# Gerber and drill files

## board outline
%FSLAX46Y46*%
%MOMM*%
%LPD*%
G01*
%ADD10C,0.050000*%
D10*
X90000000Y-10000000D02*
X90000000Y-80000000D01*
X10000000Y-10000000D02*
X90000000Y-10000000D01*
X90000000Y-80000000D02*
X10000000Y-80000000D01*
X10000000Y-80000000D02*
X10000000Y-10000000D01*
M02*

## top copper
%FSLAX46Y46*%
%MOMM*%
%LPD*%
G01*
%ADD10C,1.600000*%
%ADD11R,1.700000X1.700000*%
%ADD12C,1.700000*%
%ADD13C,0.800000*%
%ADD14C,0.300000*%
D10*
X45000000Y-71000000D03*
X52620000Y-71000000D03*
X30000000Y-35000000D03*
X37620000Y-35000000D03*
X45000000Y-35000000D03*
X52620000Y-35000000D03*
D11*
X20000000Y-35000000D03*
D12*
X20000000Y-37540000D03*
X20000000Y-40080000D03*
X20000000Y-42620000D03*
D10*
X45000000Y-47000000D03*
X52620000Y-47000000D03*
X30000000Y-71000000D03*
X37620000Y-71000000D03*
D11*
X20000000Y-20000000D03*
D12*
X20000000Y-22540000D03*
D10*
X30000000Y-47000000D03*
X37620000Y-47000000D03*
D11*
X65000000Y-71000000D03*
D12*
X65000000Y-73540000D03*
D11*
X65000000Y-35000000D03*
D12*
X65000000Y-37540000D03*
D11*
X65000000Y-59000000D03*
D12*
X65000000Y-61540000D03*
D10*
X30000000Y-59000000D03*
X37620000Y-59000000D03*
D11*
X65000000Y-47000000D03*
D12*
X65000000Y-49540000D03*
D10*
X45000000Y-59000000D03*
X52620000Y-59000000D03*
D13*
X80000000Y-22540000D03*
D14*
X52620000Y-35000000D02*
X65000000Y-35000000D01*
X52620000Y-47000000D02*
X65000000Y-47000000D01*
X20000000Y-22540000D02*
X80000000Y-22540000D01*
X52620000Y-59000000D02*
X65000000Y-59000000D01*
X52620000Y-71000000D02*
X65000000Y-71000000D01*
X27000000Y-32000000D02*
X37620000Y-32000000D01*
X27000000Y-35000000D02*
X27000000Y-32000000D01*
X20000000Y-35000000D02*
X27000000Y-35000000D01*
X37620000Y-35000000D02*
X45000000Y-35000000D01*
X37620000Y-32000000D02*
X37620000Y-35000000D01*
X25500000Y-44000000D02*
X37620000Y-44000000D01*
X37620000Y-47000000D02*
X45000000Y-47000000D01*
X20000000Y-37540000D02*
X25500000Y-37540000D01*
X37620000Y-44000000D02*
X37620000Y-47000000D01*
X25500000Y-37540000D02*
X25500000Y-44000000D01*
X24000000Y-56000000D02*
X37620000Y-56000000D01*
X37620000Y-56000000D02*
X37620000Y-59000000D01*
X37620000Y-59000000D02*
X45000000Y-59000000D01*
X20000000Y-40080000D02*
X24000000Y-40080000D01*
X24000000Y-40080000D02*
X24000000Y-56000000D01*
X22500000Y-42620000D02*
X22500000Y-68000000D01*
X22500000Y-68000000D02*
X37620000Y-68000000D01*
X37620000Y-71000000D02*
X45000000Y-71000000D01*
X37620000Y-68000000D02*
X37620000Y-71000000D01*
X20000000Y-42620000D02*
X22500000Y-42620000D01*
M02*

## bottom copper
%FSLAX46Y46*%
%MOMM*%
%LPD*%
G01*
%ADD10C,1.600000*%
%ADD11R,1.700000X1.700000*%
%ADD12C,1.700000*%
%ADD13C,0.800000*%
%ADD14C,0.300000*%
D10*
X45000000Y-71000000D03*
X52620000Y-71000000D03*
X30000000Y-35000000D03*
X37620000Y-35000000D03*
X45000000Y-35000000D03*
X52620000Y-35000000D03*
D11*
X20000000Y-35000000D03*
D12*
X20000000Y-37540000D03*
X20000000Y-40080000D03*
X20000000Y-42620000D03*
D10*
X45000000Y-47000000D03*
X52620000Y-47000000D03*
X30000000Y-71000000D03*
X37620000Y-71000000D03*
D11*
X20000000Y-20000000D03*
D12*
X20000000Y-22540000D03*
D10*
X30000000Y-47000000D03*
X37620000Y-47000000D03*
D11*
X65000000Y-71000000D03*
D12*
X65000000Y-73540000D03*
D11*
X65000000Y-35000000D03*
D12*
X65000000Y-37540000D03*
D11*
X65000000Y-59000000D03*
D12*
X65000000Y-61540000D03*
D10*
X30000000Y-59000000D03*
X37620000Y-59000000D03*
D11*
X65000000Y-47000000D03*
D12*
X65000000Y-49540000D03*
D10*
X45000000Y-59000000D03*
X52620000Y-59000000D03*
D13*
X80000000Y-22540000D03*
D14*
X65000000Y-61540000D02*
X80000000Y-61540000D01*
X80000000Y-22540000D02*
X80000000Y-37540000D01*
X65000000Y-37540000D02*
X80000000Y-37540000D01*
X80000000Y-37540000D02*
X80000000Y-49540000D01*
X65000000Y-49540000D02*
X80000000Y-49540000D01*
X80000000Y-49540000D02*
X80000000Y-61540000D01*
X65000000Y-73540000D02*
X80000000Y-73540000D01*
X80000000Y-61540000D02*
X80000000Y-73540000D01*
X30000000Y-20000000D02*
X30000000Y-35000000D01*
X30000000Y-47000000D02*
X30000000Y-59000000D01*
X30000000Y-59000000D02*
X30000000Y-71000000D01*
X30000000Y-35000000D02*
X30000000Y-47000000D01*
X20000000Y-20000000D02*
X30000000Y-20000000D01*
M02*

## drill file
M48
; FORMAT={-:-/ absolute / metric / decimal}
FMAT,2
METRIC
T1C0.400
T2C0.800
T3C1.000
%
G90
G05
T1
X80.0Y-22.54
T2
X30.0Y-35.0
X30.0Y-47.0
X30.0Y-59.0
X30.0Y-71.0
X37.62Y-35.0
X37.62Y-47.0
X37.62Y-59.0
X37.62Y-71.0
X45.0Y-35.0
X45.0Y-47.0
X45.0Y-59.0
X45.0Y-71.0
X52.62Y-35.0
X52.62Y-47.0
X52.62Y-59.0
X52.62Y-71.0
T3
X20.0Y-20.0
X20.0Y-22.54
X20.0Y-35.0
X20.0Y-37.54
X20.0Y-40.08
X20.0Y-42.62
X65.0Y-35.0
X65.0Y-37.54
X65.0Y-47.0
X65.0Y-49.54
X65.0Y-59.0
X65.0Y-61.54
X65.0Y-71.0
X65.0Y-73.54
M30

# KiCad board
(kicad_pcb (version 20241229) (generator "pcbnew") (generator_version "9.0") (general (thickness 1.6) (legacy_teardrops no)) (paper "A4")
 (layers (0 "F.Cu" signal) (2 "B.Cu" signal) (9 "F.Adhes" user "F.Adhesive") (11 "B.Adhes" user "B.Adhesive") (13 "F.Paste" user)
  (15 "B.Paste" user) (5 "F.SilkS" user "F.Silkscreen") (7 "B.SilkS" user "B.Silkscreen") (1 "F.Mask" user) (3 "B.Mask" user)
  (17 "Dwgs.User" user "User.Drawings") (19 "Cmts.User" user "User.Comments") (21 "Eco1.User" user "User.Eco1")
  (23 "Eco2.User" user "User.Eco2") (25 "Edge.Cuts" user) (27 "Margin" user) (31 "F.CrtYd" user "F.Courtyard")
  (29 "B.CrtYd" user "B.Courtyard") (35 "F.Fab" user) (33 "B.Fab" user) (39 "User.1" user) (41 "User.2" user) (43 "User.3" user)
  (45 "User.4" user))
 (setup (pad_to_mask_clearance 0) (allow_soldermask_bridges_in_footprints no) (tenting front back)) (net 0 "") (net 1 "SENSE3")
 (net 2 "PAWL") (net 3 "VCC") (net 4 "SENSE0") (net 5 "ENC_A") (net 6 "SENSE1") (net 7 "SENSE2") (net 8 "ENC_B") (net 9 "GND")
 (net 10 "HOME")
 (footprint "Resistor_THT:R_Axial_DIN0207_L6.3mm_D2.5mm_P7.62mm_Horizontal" (layer "F.Cu") (at 45 71)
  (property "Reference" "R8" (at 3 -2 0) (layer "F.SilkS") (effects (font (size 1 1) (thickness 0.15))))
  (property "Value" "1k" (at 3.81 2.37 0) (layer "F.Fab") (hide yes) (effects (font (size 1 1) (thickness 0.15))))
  (pad "1" thru_hole circle (at 0 0) (size 1.6 1.6) (drill 0.8) (layers "*.Cu" "*.Mask") (remove_unused_layers no) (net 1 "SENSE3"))
  (pad "2" thru_hole circle (at 7.62 0) (size 1.6 1.6) (drill 0.8) (layers "*.Cu" "*.Mask") (remove_unused_layers no) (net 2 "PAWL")))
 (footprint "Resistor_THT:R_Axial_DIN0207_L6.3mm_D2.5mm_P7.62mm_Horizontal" (layer "F.Cu") (at 30 35)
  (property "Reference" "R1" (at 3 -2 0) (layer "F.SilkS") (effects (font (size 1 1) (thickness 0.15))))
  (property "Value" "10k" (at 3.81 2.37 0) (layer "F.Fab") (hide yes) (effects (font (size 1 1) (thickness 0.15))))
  (pad "1" thru_hole circle (at 0 0) (size 1.6 1.6) (drill 0.8) (layers "*.Cu" "*.Mask") (remove_unused_layers no) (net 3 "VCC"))
  (pad "2" thru_hole circle (at 7.62 0) (size 1.6 1.6) (drill 0.8) (layers "*.Cu" "*.Mask") (remove_unused_layers no) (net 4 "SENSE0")))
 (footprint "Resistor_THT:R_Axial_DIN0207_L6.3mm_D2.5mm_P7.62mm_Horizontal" (layer "F.Cu") (at 45 35)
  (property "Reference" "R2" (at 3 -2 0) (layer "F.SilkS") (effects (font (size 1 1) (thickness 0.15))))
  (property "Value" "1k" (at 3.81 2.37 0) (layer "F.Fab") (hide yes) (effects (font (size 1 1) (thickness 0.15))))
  (pad "1" thru_hole circle (at 0 0) (size 1.6 1.6) (drill 0.8) (layers "*.Cu" "*.Mask") (remove_unused_layers no) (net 4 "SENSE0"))
  (pad "2" thru_hole circle (at 7.62 0) (size 1.6 1.6) (drill 0.8) (layers "*.Cu" "*.Mask") (remove_unused_layers no) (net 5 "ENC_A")))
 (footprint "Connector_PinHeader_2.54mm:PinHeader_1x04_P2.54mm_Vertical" (layer "F.Cu") (at 20 35)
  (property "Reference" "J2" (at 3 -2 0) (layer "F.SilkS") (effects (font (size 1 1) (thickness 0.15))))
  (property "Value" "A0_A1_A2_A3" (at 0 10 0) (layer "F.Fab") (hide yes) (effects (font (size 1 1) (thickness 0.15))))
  (pad "1" thru_hole rect (at 0 0) (size 1.7 1.7) (drill 1) (layers "*.Cu" "*.Mask") (remove_unused_layers no) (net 4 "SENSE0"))
  (pad "2" thru_hole circle (at 0 2.54) (size 1.7 1.7) (drill 1) (layers "*.Cu" "*.Mask") (remove_unused_layers no) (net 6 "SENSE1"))
  (pad "3" thru_hole circle (at 0 5.08) (size 1.7 1.7) (drill 1) (layers "*.Cu" "*.Mask") (remove_unused_layers no) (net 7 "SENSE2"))
  (pad "4" thru_hole circle (at 0 7.62) (size 1.7 1.7) (drill 1) (layers "*.Cu" "*.Mask") (remove_unused_layers no) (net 1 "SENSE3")))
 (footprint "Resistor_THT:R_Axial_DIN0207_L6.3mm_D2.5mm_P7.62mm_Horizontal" (layer "F.Cu") (at 45 47)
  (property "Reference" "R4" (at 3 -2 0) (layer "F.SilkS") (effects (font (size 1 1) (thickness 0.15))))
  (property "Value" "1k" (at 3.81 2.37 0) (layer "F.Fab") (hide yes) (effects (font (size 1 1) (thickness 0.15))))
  (pad "1" thru_hole circle (at 0 0) (size 1.6 1.6) (drill 0.8) (layers "*.Cu" "*.Mask") (remove_unused_layers no) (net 6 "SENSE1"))
  (pad "2" thru_hole circle (at 7.62 0) (size 1.6 1.6) (drill 0.8) (layers "*.Cu" "*.Mask") (remove_unused_layers no) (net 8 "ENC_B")))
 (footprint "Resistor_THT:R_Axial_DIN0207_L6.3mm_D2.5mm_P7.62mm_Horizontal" (layer "F.Cu") (at 30 71)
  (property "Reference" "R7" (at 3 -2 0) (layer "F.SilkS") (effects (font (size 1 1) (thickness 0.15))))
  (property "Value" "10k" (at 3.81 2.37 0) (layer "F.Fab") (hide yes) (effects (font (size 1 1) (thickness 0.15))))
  (pad "1" thru_hole circle (at 0 0) (size 1.6 1.6) (drill 0.8) (layers "*.Cu" "*.Mask") (remove_unused_layers no) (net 3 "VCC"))
  (pad "2" thru_hole circle (at 7.62 0) (size 1.6 1.6) (drill 0.8) (layers "*.Cu" "*.Mask") (remove_unused_layers no) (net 1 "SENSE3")))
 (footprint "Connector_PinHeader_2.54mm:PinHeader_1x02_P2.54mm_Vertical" (layer "F.Cu") (at 20 20)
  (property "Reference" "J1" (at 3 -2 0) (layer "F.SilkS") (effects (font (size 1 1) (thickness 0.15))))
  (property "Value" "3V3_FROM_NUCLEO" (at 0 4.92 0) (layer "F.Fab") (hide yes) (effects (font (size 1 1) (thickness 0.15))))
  (pad "1" thru_hole rect (at 0 0) (size 1.7 1.7) (drill 1) (layers "*.Cu" "*.Mask") (remove_unused_layers no) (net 3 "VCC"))
  (pad "2" thru_hole circle (at 0 2.54) (size 1.7 1.7) (drill 1) (layers "*.Cu" "*.Mask") (remove_unused_layers no) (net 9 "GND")))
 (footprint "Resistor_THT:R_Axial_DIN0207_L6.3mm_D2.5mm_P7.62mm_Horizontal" (layer "F.Cu") (at 30 47)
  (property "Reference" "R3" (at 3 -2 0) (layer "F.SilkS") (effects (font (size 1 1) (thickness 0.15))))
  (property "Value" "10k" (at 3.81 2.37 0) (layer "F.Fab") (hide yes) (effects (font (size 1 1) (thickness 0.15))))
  (pad "1" thru_hole circle (at 0 0) (size 1.6 1.6) (drill 0.8) (layers "*.Cu" "*.Mask") (remove_unused_layers no) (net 3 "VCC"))
  (pad "2" thru_hole circle (at 7.62 0) (size 1.6 1.6) (drill 0.8) (layers "*.Cu" "*.Mask") (remove_unused_layers no) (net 6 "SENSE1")))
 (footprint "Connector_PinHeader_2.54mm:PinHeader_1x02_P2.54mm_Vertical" (layer "F.Cu") (at 65 71)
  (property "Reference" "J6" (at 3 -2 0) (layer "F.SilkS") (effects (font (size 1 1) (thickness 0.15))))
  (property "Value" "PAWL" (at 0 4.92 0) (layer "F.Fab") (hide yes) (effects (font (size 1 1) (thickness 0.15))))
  (pad "1" thru_hole rect (at 0 0) (size 1.7 1.7) (drill 1) (layers "*.Cu" "*.Mask") (remove_unused_layers no) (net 2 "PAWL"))
  (pad "2" thru_hole circle (at 0 2.54) (size 1.7 1.7) (drill 1) (layers "*.Cu" "*.Mask") (remove_unused_layers no) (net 9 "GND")))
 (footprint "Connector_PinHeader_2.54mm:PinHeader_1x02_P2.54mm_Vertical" (layer "F.Cu") (at 65 35)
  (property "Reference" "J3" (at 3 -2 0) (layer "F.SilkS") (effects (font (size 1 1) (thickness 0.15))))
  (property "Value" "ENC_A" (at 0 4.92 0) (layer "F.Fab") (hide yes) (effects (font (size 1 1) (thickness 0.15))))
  (pad "1" thru_hole rect (at 0 0) (size 1.7 1.7) (drill 1) (layers "*.Cu" "*.Mask") (remove_unused_layers no) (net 5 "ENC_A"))
  (pad "2" thru_hole circle (at 0 2.54) (size 1.7 1.7) (drill 1) (layers "*.Cu" "*.Mask") (remove_unused_layers no) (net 9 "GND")))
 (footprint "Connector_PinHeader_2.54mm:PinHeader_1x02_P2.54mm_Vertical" (layer "F.Cu") (at 65 59)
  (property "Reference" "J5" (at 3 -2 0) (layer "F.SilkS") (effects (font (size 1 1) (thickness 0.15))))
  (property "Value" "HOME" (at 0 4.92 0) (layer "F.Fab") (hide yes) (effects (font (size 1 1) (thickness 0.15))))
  (pad "1" thru_hole rect (at 0 0) (size 1.7 1.7) (drill 1) (layers "*.Cu" "*.Mask") (remove_unused_layers no) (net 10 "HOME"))
  (pad "2" thru_hole circle (at 0 2.54) (size 1.7 1.7) (drill 1) (layers "*.Cu" "*.Mask") (remove_unused_layers no) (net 9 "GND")))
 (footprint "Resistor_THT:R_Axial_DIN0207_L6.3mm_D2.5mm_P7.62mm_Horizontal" (layer "F.Cu") (at 30 59)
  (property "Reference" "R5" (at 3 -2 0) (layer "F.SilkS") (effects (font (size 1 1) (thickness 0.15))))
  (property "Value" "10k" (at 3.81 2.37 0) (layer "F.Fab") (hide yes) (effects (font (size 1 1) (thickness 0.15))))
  (pad "1" thru_hole circle (at 0 0) (size 1.6 1.6) (drill 0.8) (layers "*.Cu" "*.Mask") (remove_unused_layers no) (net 3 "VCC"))
  (pad "2" thru_hole circle (at 7.62 0) (size 1.6 1.6) (drill 0.8) (layers "*.Cu" "*.Mask") (remove_unused_layers no) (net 7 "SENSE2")))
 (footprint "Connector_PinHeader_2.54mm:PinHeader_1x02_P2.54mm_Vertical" (layer "F.Cu") (at 65 47)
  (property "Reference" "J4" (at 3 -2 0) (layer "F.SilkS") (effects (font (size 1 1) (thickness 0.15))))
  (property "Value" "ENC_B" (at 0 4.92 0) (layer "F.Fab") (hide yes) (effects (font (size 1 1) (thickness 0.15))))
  (pad "1" thru_hole rect (at 0 0) (size 1.7 1.7) (drill 1) (layers "*.Cu" "*.Mask") (remove_unused_layers no) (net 8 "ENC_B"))
  (pad "2" thru_hole circle (at 0 2.54) (size 1.7 1.7) (drill 1) (layers "*.Cu" "*.Mask") (remove_unused_layers no) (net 9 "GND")))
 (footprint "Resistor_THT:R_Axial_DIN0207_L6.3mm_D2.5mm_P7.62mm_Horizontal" (layer "F.Cu") (at 45 59)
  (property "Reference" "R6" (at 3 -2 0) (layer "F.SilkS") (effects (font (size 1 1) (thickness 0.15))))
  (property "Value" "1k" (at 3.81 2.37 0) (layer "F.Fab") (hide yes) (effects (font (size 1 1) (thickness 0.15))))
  (pad "1" thru_hole circle (at 0 0) (size 1.6 1.6) (drill 0.8) (layers "*.Cu" "*.Mask") (remove_unused_layers no) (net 7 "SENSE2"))
  (pad "2" thru_hole circle (at 7.62 0) (size 1.6 1.6) (drill 0.8) (layers "*.Cu" "*.Mask") (remove_unused_layers no) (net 10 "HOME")))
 (gr_line (start 90 10) (end 90 80) (stroke (width 0.05) (type default)) (layer "Edge.Cuts"))
 (gr_line (start 10 10) (end 90 10) (stroke (width 0.05) (type default)) (layer "Edge.Cuts"))
 (gr_line (start 90 80) (end 10 80) (stroke (width 0.05) (type default)) (layer "Edge.Cuts"))
 (gr_line (start 10 80) (end 10 10) (stroke (width 0.05) (type default)) (layer "Edge.Cuts"))
 (segment (start 52.62 35) (end 65 35) (width 0.3) (layer "F.Cu") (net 5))
 (segment (start 52.62 47) (end 65 47) (width 0.3) (layer "F.Cu") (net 8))
 (segment (start 20 22.54) (end 80 22.54) (width 0.3) (layer "F.Cu") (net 9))
 (via (at 80 22.54) (size 0.8) (drill 0.4) (layers "F.Cu" "B.Cu") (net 9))
 (segment (start 65 61.54) (end 80 61.54) (width 0.3) (layer "B.Cu") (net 9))
 (segment (start 80 22.54) (end 80 37.54) (width 0.3) (layer "B.Cu") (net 9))
 (segment (start 65 37.54) (end 80 37.54) (width 0.3) (layer "B.Cu") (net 9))
 (segment (start 80 37.54) (end 80 49.54) (width 0.3) (layer "B.Cu") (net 9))
 (segment (start 65 49.54) (end 80 49.54) (width 0.3) (layer "B.Cu") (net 9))
 (segment (start 80 49.54) (end 80 61.54) (width 0.3) (layer "B.Cu") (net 9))
 (segment (start 65 73.54) (end 80 73.54) (width 0.3) (layer "B.Cu") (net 9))
 (segment (start 80 61.54) (end 80 73.54) (width 0.3) (layer "B.Cu") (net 9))
 (segment (start 52.62 59) (end 65 59) (width 0.3) (layer "F.Cu") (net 10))
 (segment (start 52.62 71) (end 65 71) (width 0.3) (layer "F.Cu") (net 2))
 (segment (start 27 32) (end 37.62 32) (width 0.3) (layer "F.Cu") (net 4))
 (segment (start 27 35) (end 27 32) (width 0.3) (layer "F.Cu") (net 4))
 (segment (start 20 35) (end 27 35) (width 0.3) (layer "F.Cu") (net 4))
 (segment (start 37.62 35) (end 45 35) (width 0.3) (layer "F.Cu") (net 4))
 (segment (start 37.62 32) (end 37.62 35) (width 0.3) (layer "F.Cu") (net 4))
 (segment (start 25.5 44) (end 37.62 44) (width 0.3) (layer "F.Cu") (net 6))
 (segment (start 37.62 47) (end 45 47) (width 0.3) (layer "F.Cu") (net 6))
 (segment (start 20 37.54) (end 25.5 37.54) (width 0.3) (layer "F.Cu") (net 6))
 (segment (start 37.62 44) (end 37.62 47) (width 0.3) (layer "F.Cu") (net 6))
 (segment (start 25.5 37.54) (end 25.5 44) (width 0.3) (layer "F.Cu") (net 6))
 (segment (start 24 56) (end 37.62 56) (width 0.3) (layer "F.Cu") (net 7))
 (segment (start 37.62 56) (end 37.62 59) (width 0.3) (layer "F.Cu") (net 7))
 (segment (start 37.62 59) (end 45 59) (width 0.3) (layer "F.Cu") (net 7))
 (segment (start 20 40.08) (end 24 40.08) (width 0.3) (layer "F.Cu") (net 7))
 (segment (start 24 40.08) (end 24 56) (width 0.3) (layer "F.Cu") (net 7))
 (segment (start 22.5 42.62) (end 22.5 68) (width 0.3) (layer "F.Cu") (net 1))
 (segment (start 22.5 68) (end 37.62 68) (width 0.3) (layer "F.Cu") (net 1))
 (segment (start 37.62 71) (end 45 71) (width 0.3) (layer "F.Cu") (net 1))
 (segment (start 37.62 68) (end 37.62 71) (width 0.3) (layer "F.Cu") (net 1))
 (segment (start 20 42.62) (end 22.5 42.62) (width 0.3) (layer "F.Cu") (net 1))
 (segment (start 30 20) (end 30 35) (width 0.3) (layer "B.Cu") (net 3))
 (segment (start 30 47) (end 30 59) (width 0.3) (layer "B.Cu") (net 3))
 (segment (start 30 59) (end 30 71) (width 0.3) (layer "B.Cu") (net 3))
 (segment (start 30 35) (end 30 47) (width 0.3) (layer "B.Cu") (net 3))
 (segment (start 20 20) (end 30 20) (width 0.3) (layer "B.Cu") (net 3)))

